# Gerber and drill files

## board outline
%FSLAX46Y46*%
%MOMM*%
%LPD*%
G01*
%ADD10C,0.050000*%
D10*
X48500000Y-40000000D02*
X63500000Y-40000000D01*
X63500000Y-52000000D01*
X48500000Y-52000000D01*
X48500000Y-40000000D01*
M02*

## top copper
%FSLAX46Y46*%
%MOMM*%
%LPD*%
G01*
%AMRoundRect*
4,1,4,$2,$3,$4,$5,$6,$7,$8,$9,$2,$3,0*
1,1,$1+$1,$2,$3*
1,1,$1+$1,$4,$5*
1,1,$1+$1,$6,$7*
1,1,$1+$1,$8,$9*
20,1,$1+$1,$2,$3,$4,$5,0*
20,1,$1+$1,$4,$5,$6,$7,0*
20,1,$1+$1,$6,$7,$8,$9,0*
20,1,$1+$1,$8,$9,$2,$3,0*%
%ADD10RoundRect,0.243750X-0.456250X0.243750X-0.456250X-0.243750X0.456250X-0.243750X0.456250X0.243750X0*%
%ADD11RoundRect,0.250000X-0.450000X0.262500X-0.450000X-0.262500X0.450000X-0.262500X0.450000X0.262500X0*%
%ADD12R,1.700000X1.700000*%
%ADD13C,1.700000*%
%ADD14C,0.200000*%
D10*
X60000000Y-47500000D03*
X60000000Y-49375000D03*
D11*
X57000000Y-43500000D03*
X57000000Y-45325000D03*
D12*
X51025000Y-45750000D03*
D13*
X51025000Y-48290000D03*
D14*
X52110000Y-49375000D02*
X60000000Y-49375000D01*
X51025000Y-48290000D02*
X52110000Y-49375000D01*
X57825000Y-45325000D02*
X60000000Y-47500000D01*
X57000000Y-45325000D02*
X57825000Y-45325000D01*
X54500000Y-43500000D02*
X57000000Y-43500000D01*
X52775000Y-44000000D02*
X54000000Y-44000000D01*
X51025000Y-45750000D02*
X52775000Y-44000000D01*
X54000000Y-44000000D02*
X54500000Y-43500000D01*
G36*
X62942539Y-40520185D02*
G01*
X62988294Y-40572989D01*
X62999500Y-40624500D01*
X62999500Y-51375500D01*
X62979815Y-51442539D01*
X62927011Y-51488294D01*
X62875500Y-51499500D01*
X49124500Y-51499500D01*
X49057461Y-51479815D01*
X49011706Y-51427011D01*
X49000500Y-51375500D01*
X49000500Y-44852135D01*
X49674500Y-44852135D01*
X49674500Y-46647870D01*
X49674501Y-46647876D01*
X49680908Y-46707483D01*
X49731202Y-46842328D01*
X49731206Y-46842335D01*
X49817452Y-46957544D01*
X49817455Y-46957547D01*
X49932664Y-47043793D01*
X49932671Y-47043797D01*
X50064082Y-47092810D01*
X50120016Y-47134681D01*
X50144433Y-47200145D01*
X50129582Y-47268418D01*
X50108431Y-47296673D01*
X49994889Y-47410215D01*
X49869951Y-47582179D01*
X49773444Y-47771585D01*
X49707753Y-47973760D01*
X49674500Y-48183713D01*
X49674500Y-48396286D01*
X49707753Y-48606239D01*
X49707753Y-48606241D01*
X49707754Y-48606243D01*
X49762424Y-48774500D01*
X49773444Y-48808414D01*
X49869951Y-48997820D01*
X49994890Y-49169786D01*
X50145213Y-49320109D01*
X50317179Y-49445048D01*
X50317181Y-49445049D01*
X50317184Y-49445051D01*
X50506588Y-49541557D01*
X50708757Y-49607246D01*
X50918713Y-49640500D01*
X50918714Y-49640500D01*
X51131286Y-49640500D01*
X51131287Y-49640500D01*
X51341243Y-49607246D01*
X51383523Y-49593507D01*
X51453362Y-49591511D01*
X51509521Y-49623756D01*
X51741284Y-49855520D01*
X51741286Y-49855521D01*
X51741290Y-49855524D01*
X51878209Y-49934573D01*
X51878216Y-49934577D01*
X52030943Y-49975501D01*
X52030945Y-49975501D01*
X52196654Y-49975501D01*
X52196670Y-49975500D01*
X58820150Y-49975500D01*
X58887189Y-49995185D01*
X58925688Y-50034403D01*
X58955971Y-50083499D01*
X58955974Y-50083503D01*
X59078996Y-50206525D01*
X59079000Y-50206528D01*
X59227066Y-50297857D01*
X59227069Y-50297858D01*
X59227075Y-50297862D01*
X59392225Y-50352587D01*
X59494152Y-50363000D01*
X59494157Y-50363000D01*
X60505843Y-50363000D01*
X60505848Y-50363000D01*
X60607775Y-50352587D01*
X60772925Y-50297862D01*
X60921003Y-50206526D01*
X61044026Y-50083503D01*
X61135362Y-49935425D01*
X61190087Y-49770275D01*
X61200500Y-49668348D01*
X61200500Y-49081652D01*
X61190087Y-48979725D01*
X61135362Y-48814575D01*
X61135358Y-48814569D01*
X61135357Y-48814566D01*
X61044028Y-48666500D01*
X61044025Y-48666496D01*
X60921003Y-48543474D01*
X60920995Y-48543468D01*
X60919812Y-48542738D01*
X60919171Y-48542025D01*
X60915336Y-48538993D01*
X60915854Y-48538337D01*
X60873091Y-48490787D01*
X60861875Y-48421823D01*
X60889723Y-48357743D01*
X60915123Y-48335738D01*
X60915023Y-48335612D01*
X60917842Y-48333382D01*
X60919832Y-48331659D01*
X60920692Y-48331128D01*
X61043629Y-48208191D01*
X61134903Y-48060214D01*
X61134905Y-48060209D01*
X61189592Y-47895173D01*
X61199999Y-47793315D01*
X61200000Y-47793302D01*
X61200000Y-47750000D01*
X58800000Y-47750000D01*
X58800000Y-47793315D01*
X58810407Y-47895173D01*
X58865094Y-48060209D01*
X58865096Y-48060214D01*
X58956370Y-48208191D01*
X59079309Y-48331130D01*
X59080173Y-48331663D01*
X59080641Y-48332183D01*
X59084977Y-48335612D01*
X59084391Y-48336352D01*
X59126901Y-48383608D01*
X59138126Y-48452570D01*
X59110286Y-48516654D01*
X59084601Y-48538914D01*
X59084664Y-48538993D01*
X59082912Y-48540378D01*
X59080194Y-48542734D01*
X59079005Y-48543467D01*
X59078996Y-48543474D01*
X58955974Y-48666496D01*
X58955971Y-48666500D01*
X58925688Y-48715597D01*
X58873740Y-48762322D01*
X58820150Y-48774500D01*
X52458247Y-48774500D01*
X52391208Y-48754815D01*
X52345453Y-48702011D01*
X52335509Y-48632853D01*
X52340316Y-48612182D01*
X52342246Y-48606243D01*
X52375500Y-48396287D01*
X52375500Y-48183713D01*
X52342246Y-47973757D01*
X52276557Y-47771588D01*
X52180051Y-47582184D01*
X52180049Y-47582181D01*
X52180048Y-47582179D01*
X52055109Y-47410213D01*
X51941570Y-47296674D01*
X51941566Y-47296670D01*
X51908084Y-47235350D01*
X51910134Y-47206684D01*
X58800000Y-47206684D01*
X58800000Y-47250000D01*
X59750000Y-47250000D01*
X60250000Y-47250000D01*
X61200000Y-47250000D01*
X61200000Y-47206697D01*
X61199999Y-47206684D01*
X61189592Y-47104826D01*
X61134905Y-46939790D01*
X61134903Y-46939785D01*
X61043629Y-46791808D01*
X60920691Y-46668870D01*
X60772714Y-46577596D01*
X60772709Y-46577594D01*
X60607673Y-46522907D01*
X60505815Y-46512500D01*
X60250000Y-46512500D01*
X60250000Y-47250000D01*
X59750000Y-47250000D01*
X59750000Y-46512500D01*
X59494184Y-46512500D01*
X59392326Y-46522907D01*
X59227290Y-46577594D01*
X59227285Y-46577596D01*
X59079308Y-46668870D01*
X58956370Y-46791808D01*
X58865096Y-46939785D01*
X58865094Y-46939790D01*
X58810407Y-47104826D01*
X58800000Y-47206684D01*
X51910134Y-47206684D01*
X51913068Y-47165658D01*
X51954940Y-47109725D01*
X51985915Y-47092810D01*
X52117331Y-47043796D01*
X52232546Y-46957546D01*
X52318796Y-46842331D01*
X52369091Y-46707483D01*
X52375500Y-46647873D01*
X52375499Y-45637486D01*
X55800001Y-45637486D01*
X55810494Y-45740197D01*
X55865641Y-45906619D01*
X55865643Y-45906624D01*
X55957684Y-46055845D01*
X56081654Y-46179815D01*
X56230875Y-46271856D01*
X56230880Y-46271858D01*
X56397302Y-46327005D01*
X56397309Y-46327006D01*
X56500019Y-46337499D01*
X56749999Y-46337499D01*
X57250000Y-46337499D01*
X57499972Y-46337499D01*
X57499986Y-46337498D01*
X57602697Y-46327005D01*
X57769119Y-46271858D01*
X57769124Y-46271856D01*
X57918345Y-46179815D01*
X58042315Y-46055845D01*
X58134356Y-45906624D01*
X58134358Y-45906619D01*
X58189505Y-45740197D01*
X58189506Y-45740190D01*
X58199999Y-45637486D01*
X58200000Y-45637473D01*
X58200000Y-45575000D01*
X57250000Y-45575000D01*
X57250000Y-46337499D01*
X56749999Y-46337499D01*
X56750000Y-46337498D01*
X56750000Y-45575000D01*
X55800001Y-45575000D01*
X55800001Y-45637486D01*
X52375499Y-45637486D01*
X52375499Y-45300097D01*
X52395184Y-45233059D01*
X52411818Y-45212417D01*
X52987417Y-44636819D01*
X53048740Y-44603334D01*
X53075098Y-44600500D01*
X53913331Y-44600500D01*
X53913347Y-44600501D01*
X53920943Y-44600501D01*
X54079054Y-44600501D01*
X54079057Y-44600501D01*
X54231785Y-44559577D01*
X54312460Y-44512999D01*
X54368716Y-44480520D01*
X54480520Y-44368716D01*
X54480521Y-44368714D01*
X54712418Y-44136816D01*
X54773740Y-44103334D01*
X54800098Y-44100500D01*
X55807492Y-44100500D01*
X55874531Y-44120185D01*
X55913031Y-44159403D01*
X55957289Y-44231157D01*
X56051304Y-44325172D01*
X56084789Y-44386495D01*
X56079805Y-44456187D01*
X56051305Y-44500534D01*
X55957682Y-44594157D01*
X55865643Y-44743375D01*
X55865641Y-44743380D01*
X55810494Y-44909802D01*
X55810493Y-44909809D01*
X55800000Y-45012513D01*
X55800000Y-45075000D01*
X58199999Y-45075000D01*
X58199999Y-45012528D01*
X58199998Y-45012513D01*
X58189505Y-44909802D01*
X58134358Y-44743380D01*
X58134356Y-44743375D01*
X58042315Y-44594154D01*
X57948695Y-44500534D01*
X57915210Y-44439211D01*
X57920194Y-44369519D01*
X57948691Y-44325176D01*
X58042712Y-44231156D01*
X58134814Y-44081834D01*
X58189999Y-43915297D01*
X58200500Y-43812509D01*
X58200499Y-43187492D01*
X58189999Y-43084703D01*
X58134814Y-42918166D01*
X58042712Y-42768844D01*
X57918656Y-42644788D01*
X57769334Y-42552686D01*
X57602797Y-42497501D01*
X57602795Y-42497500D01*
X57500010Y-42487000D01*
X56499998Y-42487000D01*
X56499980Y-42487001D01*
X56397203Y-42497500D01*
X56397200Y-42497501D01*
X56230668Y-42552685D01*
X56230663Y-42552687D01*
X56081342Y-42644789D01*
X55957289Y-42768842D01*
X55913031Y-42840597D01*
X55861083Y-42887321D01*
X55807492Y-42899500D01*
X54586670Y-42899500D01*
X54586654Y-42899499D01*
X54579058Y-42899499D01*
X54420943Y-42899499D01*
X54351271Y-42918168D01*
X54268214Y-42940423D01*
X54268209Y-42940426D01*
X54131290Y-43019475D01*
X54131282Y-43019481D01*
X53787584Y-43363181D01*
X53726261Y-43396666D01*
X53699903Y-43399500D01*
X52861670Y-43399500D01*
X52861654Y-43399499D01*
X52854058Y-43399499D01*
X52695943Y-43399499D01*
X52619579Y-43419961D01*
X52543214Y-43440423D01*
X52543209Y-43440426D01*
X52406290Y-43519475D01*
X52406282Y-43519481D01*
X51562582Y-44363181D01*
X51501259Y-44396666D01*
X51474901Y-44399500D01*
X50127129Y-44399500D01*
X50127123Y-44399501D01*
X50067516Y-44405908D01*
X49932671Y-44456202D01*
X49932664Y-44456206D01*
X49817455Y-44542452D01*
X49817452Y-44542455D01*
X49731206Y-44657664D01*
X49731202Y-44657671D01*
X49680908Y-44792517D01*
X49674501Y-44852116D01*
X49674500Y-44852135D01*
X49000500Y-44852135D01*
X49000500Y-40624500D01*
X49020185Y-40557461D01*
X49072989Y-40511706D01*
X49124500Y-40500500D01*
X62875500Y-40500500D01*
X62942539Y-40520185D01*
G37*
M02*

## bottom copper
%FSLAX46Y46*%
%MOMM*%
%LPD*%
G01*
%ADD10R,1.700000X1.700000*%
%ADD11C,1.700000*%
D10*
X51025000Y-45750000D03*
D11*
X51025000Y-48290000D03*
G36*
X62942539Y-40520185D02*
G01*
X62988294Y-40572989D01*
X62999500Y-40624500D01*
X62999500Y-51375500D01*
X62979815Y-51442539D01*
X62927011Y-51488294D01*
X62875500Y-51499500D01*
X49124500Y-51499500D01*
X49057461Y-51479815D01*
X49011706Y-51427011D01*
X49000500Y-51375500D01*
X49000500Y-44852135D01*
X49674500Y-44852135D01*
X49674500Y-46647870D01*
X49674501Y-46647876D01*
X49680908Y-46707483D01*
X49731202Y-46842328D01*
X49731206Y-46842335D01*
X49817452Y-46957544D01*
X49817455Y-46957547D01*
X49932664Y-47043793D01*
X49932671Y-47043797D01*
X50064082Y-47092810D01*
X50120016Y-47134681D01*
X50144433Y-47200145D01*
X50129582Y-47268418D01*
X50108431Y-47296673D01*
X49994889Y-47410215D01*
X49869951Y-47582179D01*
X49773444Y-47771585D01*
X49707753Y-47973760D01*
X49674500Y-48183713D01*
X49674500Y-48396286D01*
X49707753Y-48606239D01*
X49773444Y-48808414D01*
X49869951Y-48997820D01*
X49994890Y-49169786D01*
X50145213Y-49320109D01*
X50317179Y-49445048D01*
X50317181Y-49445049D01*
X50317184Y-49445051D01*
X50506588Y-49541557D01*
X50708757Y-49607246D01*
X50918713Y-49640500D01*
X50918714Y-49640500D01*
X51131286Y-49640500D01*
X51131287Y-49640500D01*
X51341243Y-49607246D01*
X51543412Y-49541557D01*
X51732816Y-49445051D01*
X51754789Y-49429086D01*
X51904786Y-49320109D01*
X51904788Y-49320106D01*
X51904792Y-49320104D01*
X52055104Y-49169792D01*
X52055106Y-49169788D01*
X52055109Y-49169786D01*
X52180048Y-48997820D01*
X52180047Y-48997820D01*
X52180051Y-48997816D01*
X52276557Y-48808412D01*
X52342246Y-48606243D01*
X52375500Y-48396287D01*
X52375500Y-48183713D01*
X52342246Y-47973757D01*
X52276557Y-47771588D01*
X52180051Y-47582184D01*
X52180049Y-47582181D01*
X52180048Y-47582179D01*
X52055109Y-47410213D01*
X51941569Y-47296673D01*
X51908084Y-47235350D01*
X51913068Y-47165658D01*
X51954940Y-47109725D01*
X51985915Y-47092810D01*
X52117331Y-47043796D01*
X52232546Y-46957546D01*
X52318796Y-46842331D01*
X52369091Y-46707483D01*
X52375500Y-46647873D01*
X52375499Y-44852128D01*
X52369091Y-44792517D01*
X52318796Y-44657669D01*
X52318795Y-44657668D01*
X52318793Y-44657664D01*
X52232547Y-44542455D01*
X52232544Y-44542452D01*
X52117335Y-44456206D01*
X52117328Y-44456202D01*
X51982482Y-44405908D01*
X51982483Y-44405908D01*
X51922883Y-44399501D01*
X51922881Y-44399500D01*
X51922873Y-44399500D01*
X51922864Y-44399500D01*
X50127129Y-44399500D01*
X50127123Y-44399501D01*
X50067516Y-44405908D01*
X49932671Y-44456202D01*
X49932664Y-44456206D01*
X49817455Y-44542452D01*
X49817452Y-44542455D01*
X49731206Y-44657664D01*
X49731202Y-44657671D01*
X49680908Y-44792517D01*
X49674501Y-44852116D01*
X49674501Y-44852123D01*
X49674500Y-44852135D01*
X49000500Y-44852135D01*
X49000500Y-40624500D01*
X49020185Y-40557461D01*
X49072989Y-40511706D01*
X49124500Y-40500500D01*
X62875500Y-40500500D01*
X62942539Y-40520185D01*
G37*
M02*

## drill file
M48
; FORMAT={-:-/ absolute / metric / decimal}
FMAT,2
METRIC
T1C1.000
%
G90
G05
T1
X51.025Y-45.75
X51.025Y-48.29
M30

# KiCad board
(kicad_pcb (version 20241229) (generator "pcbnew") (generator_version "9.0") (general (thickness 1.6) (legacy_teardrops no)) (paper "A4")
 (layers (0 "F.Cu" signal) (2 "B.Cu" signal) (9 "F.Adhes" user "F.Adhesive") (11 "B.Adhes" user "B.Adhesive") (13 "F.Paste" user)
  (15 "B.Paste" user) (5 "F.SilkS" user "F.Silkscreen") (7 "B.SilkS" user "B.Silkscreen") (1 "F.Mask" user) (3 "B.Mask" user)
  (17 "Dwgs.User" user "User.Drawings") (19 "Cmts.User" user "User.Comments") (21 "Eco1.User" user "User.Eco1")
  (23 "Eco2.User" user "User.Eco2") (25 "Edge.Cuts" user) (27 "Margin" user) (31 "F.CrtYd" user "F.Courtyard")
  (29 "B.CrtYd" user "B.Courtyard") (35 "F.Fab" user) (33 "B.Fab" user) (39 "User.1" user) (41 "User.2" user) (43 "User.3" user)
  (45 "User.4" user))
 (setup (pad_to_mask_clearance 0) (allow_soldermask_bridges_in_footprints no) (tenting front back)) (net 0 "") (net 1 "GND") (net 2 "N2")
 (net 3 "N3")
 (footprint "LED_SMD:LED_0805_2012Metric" (layer "F.Cu") (at 60 48.4375 -90)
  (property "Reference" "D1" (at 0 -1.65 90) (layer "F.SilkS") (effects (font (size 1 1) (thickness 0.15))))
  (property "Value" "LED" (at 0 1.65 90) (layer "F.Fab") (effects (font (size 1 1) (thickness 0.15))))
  (pad "1" smd roundrect (at -0.9375 0 270) (size 0.975 1.4) (layers "F.Cu" "F.Mask" "F.Paste") (roundrect_rratio 0.25) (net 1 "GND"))
  (pad "2" smd roundrect (at 0.9375 0 270) (size 0.975 1.4) (layers "F.Cu" "F.Mask" "F.Paste") (roundrect_rratio 0.25) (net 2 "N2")))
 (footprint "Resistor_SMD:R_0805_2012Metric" (layer "F.Cu") (at 57 44.4125 -90)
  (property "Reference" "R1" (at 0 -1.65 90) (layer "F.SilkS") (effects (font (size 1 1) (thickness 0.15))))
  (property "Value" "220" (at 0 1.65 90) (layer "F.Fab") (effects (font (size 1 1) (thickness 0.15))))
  (pad "1" smd roundrect (at -0.9125 0 270) (size 1.025 1.4) (layers "F.Cu" "F.Mask" "F.Paste") (roundrect_rratio 0.243902) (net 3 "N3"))
  (pad "2" smd roundrect (at 0.9125 0 270) (size 1.025 1.4) (layers "F.Cu" "F.Mask" "F.Paste") (roundrect_rratio 0.243902) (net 1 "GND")))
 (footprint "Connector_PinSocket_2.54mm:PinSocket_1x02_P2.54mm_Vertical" (layer "F.Cu") (at 51.025 45.75)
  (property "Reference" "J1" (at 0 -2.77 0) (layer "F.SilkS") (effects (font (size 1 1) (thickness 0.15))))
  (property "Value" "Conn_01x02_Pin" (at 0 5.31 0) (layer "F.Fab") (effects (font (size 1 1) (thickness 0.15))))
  (pad "1" thru_hole rect (at 0 0) (size 1.7 1.7) (drill 1) (layers "*.Cu" "*.Mask") (remove_unused_layers no) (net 3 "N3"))
  (pad "2" thru_hole circle (at 0 2.54) (size 1.7 1.7) (drill 1) (layers "*.Cu" "*.Mask") (remove_unused_layers no) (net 2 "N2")))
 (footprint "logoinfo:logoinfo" (layer "F.Cu") (at 60 45.5)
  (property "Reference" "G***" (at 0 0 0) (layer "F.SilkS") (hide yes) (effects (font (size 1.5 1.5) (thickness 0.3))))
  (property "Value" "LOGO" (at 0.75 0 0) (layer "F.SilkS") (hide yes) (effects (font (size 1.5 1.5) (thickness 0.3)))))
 (gr_rect (start 48.5 40) (end 63.5 52) (stroke (width 0.05) (type default)) (fill no) (layer "Edge.Cuts"))
 (segment (start 52.11 49.375) (end 60 49.375) (width 0.2) (layer "F.Cu") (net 2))
 (segment (start 51.025 48.29) (end 52.11 49.375) (width 0.2) (layer "F.Cu") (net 2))
 (segment (start 57.825 45.325) (end 60 47.5) (width 0.2) (layer "F.Cu") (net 1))
 (segment (start 57 45.325) (end 57.825 45.325) (width 0.2) (layer "F.Cu") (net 1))
 (segment (start 54.5 43.5) (end 57 43.5) (width 0.2) (layer "F.Cu") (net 3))
 (segment (start 52.775 44) (end 54 44) (width 0.2) (layer "F.Cu") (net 3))
 (segment (start 51.025 45.75) (end 52.775 44) (width 0.2) (layer "F.Cu") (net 3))
 (segment (start 54 44) (end 54.5 43.5) (width 0.2) (layer "F.Cu") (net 3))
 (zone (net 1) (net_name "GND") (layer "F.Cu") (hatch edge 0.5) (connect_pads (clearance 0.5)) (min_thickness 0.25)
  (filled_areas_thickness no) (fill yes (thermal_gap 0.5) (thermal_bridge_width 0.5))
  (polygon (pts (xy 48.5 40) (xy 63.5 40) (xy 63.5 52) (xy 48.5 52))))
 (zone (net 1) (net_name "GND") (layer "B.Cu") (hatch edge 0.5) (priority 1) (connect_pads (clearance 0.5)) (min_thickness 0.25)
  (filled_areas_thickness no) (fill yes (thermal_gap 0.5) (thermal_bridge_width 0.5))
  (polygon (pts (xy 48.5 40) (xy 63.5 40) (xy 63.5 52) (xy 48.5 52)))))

